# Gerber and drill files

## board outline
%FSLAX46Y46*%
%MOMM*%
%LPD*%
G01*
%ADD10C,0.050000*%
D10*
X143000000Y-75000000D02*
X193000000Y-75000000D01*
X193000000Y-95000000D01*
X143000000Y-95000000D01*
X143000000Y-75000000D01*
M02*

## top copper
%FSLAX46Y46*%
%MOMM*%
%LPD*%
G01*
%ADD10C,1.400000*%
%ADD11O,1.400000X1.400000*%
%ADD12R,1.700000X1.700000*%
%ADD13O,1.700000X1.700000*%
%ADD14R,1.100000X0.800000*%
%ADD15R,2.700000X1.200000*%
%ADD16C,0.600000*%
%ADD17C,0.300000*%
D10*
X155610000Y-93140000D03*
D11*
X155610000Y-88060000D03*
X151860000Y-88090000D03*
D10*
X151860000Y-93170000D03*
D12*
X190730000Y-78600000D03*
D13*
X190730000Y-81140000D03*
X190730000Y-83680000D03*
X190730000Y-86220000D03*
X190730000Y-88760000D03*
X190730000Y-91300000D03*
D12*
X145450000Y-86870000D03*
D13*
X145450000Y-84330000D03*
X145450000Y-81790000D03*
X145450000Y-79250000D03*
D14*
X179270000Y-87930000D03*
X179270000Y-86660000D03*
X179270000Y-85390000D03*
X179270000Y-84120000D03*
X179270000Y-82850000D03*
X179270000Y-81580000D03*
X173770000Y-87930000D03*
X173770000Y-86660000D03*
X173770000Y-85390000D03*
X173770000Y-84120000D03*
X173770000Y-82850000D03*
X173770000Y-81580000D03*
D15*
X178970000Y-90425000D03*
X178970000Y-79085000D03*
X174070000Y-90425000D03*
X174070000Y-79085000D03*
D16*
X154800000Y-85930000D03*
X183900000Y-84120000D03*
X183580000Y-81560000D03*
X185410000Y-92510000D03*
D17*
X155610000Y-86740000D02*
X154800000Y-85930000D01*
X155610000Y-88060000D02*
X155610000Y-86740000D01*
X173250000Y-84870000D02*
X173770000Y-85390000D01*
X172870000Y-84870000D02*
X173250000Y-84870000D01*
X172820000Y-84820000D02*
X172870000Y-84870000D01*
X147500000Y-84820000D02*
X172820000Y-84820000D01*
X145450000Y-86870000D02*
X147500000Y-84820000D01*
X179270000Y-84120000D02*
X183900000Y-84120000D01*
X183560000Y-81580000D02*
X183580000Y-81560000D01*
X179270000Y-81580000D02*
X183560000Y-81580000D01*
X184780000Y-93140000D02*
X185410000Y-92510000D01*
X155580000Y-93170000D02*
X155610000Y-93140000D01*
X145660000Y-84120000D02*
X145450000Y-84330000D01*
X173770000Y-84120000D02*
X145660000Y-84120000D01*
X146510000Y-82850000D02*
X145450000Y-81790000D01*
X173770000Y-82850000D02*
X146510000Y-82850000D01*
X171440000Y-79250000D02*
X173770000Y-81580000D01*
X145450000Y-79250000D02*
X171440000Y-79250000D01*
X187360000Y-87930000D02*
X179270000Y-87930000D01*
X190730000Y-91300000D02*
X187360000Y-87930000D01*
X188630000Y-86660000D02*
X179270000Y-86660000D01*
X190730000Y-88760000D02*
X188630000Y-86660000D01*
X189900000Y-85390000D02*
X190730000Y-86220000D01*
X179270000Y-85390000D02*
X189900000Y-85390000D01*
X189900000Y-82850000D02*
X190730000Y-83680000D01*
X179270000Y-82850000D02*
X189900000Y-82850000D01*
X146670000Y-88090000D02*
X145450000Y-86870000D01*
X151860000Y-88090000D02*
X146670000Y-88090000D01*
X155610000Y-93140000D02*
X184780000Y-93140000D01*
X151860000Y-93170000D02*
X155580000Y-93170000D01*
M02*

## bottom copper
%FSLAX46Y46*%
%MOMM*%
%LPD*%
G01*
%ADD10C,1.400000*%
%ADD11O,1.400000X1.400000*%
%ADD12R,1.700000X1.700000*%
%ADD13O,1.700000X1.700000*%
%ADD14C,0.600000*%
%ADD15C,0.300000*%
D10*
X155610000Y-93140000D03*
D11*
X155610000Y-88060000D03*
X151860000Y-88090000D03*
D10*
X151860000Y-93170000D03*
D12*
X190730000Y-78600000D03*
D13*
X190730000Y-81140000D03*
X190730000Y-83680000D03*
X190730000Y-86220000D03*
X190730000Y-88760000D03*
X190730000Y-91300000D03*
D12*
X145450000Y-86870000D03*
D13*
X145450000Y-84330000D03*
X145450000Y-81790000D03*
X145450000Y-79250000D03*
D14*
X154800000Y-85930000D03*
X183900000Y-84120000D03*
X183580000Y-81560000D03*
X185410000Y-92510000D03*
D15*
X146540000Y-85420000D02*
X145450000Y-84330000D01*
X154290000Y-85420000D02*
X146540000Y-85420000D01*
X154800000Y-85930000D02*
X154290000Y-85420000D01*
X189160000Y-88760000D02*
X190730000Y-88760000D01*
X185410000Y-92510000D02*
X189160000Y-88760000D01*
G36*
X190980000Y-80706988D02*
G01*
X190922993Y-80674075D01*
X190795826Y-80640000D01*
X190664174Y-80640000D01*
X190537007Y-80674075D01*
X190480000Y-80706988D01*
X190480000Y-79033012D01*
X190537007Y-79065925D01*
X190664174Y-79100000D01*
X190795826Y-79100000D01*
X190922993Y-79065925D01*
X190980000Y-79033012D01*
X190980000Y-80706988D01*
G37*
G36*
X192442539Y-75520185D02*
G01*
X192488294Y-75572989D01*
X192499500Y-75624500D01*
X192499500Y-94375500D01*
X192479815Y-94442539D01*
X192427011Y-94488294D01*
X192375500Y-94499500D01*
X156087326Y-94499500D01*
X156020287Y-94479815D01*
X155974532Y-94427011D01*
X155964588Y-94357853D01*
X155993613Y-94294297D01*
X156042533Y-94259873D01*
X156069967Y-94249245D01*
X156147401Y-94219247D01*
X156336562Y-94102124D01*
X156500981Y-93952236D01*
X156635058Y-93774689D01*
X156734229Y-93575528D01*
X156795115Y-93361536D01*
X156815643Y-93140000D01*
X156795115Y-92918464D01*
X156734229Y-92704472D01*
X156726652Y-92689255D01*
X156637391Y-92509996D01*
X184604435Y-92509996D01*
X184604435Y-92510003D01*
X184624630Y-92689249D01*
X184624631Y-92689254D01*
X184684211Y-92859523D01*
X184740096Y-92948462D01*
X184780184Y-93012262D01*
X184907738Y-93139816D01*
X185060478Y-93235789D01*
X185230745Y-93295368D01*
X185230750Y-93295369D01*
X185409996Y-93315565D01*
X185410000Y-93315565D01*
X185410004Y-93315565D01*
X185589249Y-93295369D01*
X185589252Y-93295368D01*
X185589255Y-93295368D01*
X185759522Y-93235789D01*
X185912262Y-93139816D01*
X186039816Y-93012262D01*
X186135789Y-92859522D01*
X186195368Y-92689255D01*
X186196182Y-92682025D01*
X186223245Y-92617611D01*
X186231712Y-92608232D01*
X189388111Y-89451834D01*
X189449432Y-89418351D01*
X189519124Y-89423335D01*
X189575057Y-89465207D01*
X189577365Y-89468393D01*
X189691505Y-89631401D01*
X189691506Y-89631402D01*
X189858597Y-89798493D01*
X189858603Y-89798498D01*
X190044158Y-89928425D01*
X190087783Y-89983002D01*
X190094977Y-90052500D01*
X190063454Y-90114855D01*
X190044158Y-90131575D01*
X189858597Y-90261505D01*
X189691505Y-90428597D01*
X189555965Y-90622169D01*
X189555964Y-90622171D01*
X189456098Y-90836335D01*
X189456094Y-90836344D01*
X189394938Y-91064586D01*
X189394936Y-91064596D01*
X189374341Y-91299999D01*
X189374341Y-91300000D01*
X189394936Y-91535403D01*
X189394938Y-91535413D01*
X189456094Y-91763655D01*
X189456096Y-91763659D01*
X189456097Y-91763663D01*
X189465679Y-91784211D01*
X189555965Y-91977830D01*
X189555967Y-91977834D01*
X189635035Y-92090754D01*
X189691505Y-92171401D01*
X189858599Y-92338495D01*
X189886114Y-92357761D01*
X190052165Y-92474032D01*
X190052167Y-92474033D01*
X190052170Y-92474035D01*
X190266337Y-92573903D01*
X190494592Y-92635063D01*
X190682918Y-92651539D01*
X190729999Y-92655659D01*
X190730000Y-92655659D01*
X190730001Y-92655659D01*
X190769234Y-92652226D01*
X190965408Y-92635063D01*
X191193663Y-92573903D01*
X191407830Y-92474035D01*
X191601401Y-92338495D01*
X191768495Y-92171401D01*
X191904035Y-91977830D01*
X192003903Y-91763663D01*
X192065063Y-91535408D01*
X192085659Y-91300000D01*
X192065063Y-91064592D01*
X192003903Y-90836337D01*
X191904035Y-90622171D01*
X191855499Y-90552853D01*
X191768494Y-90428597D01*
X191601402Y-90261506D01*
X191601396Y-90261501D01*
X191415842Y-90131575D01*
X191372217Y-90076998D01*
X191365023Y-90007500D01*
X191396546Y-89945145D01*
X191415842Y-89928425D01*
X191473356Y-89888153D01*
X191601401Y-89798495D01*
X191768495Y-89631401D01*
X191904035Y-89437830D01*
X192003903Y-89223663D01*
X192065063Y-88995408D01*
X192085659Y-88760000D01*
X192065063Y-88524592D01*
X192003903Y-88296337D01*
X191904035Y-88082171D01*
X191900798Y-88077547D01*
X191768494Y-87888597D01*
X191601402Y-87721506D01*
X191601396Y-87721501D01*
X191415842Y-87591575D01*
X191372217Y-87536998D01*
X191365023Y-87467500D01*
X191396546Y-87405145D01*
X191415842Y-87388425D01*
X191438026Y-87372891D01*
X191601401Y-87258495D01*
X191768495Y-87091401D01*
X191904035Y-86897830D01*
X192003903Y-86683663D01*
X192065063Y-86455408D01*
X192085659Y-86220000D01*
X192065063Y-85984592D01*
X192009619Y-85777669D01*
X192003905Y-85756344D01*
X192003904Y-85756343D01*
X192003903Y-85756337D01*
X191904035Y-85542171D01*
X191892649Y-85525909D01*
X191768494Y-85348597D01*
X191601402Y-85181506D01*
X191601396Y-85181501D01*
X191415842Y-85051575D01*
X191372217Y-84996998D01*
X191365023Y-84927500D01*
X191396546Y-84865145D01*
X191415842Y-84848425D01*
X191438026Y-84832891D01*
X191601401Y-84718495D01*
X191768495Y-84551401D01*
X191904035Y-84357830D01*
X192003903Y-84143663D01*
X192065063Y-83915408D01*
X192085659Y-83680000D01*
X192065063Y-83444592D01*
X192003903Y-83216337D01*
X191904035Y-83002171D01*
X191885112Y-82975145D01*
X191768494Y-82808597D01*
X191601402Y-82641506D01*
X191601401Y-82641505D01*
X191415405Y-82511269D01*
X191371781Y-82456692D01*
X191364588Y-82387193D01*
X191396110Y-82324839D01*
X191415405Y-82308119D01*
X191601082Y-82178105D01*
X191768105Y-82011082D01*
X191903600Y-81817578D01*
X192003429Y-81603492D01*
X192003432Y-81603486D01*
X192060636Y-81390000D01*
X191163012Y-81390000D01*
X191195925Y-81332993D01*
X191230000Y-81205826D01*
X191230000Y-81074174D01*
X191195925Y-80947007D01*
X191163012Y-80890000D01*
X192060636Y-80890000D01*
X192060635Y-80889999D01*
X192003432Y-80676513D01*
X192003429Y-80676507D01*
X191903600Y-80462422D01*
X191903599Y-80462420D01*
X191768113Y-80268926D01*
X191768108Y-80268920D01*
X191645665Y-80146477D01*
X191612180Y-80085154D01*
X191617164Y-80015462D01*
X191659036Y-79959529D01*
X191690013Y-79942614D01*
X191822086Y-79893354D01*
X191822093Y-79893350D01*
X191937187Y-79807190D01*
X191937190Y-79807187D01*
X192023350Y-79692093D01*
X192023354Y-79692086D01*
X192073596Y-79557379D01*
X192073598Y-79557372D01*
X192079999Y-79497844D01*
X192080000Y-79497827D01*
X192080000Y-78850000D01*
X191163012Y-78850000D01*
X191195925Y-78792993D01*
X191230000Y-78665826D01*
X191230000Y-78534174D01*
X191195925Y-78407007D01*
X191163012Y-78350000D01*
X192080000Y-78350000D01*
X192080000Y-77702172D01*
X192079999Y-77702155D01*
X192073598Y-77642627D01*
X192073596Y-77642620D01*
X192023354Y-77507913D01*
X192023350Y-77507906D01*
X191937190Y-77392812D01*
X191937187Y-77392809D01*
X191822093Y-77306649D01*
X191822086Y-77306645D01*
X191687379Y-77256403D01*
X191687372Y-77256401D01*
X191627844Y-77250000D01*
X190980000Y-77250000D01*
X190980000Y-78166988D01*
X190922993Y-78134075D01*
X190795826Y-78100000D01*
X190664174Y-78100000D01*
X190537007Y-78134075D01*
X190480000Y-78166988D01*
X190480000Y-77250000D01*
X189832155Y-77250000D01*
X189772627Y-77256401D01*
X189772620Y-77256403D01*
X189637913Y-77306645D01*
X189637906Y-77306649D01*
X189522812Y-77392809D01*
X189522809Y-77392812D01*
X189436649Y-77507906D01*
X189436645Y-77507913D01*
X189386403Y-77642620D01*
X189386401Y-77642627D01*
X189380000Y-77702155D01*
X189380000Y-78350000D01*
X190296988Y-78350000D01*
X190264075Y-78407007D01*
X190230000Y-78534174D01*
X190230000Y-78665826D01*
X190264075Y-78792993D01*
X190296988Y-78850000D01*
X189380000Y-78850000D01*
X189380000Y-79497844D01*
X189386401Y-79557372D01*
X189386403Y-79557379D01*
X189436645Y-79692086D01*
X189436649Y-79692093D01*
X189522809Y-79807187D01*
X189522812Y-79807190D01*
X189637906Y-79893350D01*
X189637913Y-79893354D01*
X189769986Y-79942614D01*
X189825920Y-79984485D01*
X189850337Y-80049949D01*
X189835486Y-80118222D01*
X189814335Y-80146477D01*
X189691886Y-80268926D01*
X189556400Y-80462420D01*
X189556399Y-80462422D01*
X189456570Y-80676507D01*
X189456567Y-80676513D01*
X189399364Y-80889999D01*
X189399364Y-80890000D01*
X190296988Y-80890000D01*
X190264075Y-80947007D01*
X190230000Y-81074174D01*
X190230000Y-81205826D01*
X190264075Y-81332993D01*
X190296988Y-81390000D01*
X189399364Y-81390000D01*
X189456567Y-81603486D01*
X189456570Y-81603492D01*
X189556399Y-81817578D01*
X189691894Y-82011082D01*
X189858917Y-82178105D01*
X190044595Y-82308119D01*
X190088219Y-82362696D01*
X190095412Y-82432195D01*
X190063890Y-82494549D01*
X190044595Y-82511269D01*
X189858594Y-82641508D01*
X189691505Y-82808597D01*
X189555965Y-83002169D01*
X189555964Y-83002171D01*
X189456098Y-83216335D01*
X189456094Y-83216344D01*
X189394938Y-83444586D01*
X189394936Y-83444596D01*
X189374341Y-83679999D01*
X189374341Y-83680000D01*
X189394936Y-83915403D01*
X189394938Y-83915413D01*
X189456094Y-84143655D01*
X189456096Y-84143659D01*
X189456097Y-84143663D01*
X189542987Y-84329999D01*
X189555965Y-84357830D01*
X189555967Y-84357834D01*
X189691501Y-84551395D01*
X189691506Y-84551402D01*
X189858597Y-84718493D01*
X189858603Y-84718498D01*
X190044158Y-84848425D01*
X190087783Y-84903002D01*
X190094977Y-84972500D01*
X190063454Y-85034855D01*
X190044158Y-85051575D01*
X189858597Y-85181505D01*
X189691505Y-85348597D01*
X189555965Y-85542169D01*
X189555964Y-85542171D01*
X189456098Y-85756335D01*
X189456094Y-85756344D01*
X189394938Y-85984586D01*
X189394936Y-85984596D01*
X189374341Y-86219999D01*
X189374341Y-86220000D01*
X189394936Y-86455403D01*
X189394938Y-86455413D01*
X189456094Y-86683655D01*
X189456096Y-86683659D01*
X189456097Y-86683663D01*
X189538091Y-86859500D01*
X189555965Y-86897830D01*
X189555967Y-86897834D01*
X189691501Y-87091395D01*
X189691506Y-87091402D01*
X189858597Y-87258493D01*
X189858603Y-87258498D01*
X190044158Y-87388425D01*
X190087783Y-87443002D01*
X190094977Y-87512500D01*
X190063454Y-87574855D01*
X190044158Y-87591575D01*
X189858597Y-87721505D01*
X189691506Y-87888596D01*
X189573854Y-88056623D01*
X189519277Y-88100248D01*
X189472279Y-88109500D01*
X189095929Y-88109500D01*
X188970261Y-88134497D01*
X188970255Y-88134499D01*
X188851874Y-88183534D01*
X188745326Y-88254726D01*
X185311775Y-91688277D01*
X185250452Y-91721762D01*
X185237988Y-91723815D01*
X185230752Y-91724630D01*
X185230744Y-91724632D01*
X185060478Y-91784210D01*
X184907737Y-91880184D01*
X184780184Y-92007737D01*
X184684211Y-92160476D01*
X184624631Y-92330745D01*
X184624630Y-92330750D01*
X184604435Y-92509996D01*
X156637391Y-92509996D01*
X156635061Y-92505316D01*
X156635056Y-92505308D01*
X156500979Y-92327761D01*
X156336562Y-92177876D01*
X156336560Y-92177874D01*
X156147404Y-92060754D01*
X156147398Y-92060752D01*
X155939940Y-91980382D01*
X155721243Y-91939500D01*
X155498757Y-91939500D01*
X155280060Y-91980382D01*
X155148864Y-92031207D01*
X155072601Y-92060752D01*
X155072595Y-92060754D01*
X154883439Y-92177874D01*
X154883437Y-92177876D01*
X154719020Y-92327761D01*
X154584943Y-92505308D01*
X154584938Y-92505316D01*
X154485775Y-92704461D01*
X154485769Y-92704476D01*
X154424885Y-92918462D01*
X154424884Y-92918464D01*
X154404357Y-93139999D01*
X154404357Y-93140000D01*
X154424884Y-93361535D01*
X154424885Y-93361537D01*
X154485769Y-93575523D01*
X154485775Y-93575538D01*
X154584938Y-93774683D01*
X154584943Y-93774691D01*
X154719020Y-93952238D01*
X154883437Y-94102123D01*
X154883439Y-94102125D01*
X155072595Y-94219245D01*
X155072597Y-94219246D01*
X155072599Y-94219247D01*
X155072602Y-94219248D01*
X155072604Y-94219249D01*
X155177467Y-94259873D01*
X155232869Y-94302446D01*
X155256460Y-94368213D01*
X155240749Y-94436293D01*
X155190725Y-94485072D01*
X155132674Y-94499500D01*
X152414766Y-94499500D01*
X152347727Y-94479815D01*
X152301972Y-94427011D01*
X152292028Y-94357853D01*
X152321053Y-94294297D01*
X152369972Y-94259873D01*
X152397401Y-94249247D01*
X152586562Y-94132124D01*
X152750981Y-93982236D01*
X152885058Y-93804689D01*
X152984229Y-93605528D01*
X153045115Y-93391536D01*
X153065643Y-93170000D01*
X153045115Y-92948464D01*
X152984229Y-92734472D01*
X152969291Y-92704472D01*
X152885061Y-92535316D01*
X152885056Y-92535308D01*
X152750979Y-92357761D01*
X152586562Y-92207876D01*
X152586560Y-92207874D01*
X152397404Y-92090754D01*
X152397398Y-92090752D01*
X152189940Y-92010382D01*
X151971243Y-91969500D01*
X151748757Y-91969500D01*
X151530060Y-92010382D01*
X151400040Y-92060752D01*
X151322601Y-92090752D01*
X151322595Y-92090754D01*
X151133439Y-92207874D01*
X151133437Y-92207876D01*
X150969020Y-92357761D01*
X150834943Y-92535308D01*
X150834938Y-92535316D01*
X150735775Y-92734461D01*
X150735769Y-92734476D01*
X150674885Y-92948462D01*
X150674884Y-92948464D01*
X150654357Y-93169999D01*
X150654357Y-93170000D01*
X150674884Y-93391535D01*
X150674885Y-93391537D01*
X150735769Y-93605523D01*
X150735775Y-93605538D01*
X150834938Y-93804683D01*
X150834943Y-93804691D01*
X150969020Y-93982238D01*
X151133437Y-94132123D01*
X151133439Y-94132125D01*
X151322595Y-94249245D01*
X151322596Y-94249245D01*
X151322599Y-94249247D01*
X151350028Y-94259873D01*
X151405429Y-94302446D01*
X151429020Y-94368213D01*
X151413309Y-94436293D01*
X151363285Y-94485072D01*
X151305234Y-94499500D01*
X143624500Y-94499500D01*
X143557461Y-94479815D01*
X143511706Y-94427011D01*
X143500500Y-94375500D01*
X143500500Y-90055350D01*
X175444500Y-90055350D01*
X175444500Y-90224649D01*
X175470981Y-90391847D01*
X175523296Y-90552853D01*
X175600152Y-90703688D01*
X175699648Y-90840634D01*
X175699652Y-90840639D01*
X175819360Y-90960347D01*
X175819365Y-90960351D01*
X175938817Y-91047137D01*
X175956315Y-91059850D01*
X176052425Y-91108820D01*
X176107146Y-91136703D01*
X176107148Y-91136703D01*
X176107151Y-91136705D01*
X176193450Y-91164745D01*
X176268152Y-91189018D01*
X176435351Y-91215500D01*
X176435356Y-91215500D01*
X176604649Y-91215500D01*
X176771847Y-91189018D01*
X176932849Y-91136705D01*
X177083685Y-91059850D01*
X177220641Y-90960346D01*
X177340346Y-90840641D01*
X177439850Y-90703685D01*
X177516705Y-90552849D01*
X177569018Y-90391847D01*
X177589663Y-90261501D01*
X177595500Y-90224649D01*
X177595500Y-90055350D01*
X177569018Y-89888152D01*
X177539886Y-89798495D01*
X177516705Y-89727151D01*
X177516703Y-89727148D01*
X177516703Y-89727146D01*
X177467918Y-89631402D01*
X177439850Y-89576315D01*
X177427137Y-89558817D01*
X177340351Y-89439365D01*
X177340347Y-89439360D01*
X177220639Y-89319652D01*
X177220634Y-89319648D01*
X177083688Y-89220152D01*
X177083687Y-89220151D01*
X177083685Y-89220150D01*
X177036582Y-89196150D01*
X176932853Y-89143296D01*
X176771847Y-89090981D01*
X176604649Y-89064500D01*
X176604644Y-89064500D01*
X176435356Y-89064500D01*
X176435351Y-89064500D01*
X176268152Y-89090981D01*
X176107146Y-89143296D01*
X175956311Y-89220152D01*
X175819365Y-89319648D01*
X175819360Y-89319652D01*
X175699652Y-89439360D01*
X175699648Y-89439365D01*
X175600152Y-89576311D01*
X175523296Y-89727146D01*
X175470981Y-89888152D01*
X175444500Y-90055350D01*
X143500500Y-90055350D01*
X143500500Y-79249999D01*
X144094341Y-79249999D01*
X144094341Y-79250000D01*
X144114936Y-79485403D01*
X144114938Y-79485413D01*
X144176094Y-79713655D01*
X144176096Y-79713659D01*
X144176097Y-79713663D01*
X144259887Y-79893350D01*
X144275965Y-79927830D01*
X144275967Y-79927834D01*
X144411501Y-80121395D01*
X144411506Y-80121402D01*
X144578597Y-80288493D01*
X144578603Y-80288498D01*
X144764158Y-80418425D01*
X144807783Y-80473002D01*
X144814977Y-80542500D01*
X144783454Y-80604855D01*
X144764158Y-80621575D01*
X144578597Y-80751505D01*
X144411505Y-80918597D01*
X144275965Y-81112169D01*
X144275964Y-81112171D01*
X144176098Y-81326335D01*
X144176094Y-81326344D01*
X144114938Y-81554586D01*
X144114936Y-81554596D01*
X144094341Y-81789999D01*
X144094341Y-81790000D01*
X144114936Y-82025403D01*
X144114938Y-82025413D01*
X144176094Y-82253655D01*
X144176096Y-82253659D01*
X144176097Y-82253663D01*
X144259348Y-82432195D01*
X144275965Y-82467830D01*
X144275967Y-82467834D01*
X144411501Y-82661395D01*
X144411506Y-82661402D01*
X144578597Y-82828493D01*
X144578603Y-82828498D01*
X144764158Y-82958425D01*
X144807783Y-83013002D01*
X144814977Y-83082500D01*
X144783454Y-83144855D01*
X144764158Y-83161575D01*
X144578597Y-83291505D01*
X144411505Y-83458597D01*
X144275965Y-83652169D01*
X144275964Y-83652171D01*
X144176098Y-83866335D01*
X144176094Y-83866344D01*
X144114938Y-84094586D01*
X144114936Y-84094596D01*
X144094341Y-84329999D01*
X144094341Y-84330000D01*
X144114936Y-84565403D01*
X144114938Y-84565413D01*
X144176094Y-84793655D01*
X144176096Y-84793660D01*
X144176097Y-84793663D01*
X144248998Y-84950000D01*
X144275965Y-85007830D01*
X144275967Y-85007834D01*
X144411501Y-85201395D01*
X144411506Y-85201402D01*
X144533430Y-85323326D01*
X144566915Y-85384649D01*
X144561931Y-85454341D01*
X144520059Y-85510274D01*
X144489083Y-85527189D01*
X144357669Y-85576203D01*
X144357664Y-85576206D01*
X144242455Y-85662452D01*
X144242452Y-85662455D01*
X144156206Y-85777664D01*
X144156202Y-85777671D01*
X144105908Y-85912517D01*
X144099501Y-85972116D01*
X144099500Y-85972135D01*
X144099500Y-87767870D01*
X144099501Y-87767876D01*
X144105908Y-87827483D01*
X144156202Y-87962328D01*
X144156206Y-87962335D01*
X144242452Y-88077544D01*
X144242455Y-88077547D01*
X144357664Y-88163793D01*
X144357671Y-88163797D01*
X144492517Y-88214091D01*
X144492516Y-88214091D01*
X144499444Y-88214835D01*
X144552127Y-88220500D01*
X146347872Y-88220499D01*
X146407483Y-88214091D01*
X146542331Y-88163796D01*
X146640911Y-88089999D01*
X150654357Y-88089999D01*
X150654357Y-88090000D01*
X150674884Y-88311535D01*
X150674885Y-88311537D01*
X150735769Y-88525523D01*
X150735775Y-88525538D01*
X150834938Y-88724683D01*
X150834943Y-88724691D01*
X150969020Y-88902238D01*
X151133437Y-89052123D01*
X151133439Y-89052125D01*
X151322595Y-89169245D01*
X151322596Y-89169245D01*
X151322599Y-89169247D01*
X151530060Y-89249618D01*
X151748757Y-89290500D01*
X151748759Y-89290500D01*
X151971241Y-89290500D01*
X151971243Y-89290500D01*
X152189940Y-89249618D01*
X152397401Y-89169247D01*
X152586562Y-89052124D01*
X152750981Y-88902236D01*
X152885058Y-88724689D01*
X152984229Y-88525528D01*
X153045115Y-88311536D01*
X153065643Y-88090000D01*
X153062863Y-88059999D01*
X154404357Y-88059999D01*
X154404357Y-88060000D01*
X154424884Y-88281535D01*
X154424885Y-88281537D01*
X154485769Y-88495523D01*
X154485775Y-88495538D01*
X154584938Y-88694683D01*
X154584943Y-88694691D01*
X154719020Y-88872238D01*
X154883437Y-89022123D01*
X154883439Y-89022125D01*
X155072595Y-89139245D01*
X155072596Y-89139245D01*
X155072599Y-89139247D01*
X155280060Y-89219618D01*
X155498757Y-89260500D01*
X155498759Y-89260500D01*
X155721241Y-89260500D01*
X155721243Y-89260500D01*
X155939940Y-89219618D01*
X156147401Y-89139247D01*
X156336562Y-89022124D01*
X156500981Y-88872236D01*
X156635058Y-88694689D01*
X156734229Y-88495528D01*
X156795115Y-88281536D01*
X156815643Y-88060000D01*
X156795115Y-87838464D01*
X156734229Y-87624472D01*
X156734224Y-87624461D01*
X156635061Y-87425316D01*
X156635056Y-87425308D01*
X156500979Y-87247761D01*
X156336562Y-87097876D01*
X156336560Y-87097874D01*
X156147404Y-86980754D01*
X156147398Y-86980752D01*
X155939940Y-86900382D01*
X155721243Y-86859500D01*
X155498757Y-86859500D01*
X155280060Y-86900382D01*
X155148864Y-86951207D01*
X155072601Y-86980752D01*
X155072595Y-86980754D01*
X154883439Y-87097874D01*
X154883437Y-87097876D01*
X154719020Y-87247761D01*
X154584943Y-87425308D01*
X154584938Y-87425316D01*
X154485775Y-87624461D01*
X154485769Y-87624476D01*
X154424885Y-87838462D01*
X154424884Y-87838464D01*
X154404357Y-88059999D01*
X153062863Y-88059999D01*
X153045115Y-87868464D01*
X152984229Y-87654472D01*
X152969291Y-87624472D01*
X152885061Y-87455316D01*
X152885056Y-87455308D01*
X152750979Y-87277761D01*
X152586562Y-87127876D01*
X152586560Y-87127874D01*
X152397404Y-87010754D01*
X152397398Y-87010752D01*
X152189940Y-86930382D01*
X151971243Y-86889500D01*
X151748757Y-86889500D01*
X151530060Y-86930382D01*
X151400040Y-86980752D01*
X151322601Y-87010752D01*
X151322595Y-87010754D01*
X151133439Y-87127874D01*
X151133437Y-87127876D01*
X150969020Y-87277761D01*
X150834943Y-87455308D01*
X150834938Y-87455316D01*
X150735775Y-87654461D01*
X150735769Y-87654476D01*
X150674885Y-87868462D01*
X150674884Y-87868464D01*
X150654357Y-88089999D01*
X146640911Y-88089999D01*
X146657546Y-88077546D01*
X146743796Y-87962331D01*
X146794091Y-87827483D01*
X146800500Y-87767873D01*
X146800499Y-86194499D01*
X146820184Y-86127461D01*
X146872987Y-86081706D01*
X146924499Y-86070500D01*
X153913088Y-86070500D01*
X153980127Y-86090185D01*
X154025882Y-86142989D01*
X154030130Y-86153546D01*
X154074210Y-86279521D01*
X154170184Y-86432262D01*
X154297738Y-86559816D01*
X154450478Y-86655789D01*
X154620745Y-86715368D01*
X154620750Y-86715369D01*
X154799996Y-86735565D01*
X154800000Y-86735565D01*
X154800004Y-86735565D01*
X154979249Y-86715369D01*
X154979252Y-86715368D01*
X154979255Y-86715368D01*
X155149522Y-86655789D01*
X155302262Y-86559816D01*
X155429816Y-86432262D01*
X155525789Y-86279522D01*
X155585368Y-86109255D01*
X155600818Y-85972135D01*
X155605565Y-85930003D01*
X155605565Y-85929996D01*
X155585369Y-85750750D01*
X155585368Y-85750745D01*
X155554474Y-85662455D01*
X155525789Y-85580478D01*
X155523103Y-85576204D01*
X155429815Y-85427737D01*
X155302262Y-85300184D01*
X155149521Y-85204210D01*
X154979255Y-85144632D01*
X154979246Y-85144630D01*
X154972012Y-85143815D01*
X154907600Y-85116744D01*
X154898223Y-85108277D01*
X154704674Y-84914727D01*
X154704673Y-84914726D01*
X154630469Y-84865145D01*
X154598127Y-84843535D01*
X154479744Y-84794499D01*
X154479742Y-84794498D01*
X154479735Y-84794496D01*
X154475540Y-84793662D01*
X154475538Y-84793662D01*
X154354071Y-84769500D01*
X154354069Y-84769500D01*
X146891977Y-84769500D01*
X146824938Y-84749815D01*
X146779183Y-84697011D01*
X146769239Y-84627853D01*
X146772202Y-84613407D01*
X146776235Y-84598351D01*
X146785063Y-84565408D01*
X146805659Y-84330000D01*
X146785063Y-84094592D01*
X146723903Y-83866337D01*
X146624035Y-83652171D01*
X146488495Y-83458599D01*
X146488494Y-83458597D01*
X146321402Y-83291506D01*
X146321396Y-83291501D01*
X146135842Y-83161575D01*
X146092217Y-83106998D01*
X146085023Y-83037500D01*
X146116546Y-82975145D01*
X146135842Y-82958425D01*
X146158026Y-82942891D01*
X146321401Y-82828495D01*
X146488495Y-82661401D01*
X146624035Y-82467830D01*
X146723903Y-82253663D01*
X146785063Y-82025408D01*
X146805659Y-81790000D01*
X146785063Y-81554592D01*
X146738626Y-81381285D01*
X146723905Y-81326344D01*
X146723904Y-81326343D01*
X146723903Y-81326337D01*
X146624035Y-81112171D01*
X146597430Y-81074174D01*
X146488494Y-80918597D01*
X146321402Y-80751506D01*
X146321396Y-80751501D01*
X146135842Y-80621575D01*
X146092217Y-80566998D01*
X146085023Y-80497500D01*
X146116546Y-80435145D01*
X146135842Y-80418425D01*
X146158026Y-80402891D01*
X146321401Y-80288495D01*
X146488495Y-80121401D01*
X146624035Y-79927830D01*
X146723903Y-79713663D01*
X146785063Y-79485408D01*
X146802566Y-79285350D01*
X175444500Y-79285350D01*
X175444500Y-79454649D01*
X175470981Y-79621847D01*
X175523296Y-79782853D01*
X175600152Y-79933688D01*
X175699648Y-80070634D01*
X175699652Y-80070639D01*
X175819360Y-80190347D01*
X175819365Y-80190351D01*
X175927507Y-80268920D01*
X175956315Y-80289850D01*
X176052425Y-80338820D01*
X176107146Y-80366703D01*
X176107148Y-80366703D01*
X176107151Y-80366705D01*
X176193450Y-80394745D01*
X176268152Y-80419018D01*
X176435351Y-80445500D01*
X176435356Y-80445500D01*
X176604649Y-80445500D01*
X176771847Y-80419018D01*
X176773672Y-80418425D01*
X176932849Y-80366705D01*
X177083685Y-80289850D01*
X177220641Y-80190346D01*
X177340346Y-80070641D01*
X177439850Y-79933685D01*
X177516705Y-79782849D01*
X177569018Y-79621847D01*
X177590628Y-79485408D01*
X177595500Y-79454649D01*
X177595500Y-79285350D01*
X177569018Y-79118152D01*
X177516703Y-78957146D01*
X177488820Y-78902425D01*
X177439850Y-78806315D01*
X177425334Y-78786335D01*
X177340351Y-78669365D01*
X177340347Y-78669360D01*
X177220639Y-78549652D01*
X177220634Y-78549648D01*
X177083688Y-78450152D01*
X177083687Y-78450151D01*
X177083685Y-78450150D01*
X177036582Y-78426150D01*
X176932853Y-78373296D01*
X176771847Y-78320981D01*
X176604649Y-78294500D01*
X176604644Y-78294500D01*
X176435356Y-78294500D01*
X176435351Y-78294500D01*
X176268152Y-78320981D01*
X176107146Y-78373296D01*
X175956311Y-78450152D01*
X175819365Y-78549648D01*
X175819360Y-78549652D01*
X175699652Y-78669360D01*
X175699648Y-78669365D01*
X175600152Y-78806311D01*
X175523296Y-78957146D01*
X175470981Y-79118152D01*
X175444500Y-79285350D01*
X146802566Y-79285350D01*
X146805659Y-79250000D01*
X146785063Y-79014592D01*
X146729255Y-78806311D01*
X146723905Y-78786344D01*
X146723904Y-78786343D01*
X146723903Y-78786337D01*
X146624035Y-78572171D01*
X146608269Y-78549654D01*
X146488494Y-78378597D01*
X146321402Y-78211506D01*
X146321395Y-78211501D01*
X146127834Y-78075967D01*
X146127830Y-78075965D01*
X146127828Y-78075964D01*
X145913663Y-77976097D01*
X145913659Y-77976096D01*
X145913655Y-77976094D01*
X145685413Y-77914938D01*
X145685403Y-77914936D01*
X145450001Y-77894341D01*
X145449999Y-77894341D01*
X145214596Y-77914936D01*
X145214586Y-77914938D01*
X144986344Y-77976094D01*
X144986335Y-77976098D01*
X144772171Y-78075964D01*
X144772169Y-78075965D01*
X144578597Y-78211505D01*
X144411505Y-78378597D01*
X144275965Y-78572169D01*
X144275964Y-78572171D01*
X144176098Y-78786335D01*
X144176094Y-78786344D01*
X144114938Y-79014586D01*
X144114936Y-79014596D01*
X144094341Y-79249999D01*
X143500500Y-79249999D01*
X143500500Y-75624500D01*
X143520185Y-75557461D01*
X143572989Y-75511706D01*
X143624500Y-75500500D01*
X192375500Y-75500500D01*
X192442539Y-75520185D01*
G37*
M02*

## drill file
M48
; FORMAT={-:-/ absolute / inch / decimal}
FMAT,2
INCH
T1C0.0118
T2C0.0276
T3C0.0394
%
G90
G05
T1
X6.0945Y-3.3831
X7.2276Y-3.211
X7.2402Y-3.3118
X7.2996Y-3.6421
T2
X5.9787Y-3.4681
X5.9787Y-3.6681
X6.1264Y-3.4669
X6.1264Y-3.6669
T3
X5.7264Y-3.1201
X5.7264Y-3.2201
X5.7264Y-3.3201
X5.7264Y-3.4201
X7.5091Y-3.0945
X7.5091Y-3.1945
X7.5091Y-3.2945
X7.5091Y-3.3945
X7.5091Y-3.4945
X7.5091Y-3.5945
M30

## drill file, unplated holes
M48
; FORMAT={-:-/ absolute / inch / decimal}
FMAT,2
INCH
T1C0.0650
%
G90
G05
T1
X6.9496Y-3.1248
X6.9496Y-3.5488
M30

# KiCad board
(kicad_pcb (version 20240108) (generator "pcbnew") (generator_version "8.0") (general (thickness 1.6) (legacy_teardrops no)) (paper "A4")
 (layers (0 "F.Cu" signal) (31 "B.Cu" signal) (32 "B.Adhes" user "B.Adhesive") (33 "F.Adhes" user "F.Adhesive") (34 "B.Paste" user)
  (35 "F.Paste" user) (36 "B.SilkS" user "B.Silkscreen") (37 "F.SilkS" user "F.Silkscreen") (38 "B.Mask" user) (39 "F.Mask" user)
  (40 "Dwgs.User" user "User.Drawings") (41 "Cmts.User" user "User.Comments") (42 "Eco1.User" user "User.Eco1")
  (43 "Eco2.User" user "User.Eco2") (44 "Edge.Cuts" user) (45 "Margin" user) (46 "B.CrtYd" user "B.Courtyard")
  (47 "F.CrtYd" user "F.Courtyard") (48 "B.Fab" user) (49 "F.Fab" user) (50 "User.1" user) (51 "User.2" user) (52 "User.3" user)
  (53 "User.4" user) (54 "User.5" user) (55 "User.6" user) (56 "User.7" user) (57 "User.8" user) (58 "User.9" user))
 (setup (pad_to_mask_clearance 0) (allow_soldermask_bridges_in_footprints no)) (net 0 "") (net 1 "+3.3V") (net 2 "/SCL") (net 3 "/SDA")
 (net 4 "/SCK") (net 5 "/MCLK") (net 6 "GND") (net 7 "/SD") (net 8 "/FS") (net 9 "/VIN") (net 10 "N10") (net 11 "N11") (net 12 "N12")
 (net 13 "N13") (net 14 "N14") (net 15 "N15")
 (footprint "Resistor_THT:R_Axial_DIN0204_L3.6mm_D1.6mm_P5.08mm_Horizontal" (layer "F.Cu") (at 151.86 93.17 90)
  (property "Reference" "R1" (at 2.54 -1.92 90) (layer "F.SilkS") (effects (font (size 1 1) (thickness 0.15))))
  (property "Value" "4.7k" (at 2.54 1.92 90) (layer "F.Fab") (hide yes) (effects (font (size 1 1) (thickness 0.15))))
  (pad "1" thru_hole circle (at 0 0 90) (size 1.4 1.4) (drill 0.7) (layers "*.Cu" "*.Mask") (remove_unused_layers no) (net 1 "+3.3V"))
  (pad "2" thru_hole oval (at 5.08 0 90) (size 1.4 1.4) (drill 0.7) (layers "*.Cu" "*.Mask") (remove_unused_layers no) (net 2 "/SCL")))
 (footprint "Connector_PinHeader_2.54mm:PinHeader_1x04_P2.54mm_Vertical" (layer "F.Cu") (at 145.45 86.87 180)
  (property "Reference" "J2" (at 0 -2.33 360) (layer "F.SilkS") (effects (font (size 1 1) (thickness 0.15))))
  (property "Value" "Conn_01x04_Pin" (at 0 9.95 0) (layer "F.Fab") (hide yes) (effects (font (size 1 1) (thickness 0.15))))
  (pad "1" thru_hole rect (at 0 0 180) (size 1.7 1.7) (drill 1) (layers "*.Cu" "*.Mask") (remove_unused_layers no) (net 2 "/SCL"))
  (pad "2" thru_hole oval (at 0 2.54 180) (size 1.7 1.7) (drill 1) (layers "*.Cu" "*.Mask") (remove_unused_layers no) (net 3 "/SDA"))
  (pad "3" thru_hole oval (at 0 5.08 180) (size 1.7 1.7) (drill 1) (layers "*.Cu" "*.Mask") (remove_unused_layers no) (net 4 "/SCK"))
  (pad "4" thru_hole oval (at 0 7.62 180) (size 1.7 1.7) (drill 1) (layers "*.Cu" "*.Mask") (remove_unused_layers no) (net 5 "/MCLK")))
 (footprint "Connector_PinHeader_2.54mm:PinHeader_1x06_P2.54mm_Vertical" (layer "F.Cu") (at 190.73 78.6)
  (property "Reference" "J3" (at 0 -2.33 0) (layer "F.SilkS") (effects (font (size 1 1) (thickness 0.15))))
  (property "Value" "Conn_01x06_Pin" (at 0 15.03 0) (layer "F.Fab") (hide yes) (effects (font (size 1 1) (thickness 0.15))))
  (pad "1" thru_hole rect (at 0 0) (size 1.7 1.7) (drill 1) (layers "*.Cu" "*.Mask") (remove_unused_layers no) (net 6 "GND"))
  (pad "2" thru_hole oval (at 0 2.54) (size 1.7 1.7) (drill 1) (layers "*.Cu" "*.Mask") (remove_unused_layers no) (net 6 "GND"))
  (pad "3" thru_hole oval (at 0 5.08) (size 1.7 1.7) (drill 1) (layers "*.Cu" "*.Mask") (remove_unused_layers no) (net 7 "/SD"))
  (pad "4" thru_hole oval (at 0 7.62) (size 1.7 1.7) (drill 1) (layers "*.Cu" "*.Mask") (remove_unused_layers no) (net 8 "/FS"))
  (pad "5" thru_hole oval (at 0 10.16) (size 1.7 1.7) (drill 1) (layers "*.Cu" "*.Mask") (remove_unused_layers no) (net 1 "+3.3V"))
  (pad "6" thru_hole oval (at 0 12.7) (size 1.7 1.7) (drill 1) (layers "*.Cu" "*.Mask") (remove_unused_layers no) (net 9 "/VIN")))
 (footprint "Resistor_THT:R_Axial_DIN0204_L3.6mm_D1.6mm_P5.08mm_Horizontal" (layer "F.Cu") (at 155.61 93.14 90)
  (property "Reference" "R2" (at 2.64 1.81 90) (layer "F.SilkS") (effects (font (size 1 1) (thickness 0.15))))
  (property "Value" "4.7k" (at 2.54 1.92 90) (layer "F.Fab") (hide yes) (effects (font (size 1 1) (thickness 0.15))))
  (pad "1" thru_hole circle (at 0 0 90) (size 1.4 1.4) (drill 0.7) (layers "*.Cu" "*.Mask") (remove_unused_layers no) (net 1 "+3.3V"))
  (pad "2" thru_hole oval (at 5.08 0 90) (size 1.4 1.4) (drill 0.7) (layers "*.Cu" "*.Mask") (remove_unused_layers no) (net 3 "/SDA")))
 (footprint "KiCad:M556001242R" (layer "F.Cu") (at 176.52 84.755 90)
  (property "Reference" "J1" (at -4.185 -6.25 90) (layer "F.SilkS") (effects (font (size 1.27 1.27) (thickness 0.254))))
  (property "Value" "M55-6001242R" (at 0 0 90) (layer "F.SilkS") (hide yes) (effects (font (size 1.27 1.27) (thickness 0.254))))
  (pad "" np_thru_hole circle (at -5.385 0 90) (size 1.65 1.65) (drill 1.65) (layers "*.Cu" "*.Mask"))
  (pad "" np_thru_hole circle (at 5.385 0 90) (size 1.65 1.65) (drill 1.65) (layers "*.Cu" "*.Mask"))
  (pad "A1" smd rect (at -3.175 2.75 90) (size 0.8 1.1) (layers "F.Cu" "F.Paste" "F.Mask") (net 9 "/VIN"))
  (pad "A2" smd rect (at -1.905 2.75 90) (size 0.8 1.1) (layers "F.Cu" "F.Paste" "F.Mask") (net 1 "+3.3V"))
  (pad "A3" smd rect (at -0.635 2.75 90) (size 0.8 1.1) (layers "F.Cu" "F.Paste" "F.Mask") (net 8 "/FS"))
  (pad "A4" smd rect (at 0.635 2.75 90) (size 0.8 1.1) (layers "F.Cu" "F.Paste" "F.Mask") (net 6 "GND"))
  (pad "A5" smd rect (at 1.905 2.75 90) (size 0.8 1.1) (layers "F.Cu" "F.Paste" "F.Mask") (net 7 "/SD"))
  (pad "A6" smd rect (at 3.175 2.75 90) (size 0.8 1.1) (layers "F.Cu" "F.Paste" "F.Mask") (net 6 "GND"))
  (pad "B1" smd rect (at -3.175 -2.75 90) (size 0.8 1.1) (layers "F.Cu" "F.Paste" "F.Mask") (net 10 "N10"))
  (pad "B2" smd rect (at -1.905 -2.75 90) (size 0.8 1.1) (layers "F.Cu" "F.Paste" "F.Mask") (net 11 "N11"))
  (pad "B3" smd rect (at -0.635 -2.75 90) (size 0.8 1.1) (layers "F.Cu" "F.Paste" "F.Mask") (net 2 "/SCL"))
  (pad "B4" smd rect (at 0.635 -2.75 90) (size 0.8 1.1) (layers "F.Cu" "F.Paste" "F.Mask") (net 3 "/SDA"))
  (pad "B5" smd rect (at 1.905 -2.75 90) (size 0.8 1.1) (layers "F.Cu" "F.Paste" "F.Mask") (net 4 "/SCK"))
  (pad "B6" smd rect (at 3.175 -2.75 90) (size 0.8 1.1) (layers "F.Cu" "F.Paste" "F.Mask") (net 5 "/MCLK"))
  (pad "MP1" smd rect (at -5.67 2.45 90) (size 1.2 2.7) (layers "F.Cu" "F.Paste" "F.Mask") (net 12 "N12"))
  (pad "MP2" smd rect (at 5.67 2.45 90) (size 1.2 2.7) (layers "F.Cu" "F.Paste" "F.Mask") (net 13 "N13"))
  (pad "MP3" smd rect (at -5.67 -2.45 90) (size 1.2 2.7) (layers "F.Cu" "F.Paste" "F.Mask") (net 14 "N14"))
  (pad "MP4" smd rect (at 5.67 -2.45 90) (size 1.2 2.7) (layers "F.Cu" "F.Paste" "F.Mask") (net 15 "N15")))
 (gr_rect (start 143 75) (end 193 95) (stroke (width 0.05) (type default)) (fill none) (layer "Edge.Cuts"))
 (segment (start 146.51 82.85) (end 145.45 81.79) (width 0.3) (layer "F.Cu") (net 4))
 (segment (start 173.77 82.85) (end 146.51 82.85) (width 0.3) (layer "F.Cu") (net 4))
 (segment (start 179.27 81.58) (end 183.56 81.58) (width 0.3) (layer "F.Cu") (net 6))
 (segment (start 179.27 84.12) (end 183.9 84.12) (width 0.3) (layer "F.Cu") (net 6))
 (segment (start 183.56 81.58) (end 183.58 81.56) (width 0.3) (layer "F.Cu") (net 6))
 (via (at 183.9 84.12) (size 0.6) (drill 0.3) (layers "F.Cu" "B.Cu") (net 6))
 (via (at 183.58 81.56) (size 0.6) (drill 0.3) (layers "F.Cu" "B.Cu") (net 6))
 (segment (start 187.36 87.93) (end 179.27 87.93) (width 0.3) (layer "F.Cu") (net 9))
 (segment (start 190.73 91.3) (end 187.36 87.93) (width 0.3) (layer "F.Cu") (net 9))
 (segment (start 189.9 85.39) (end 190.73 86.22) (width 0.3) (layer "F.Cu") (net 8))
 (segment (start 179.27 85.39) (end 189.9 85.39) (width 0.3) (layer "F.Cu") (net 8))
 (segment (start 155.61 88.06) (end 155.61 86.74) (width 0.3) (layer "F.Cu") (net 3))
 (segment (start 155.61 86.74) (end 154.8 85.93) (width 0.3) (layer "F.Cu") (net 3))
 (segment (start 145.66 84.12) (end 145.45 84.33) (width 0.3) (layer "F.Cu") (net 3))
 (segment (start 173.77 84.12) (end 145.66 84.12) (width 0.3) (layer "F.Cu") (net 3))
 (via (at 154.8 85.93) (size 0.6) (drill 0.3) (layers "F.Cu" "B.Cu") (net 3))
 (segment (start 154.29 85.42) (end 146.54 85.42) (width 0.3) (layer "B.Cu") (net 3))
 (segment (start 154.8 85.93) (end 154.29 85.42) (width 0.3) (layer "B.Cu") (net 3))
 (segment (start 146.54 85.42) (end 145.45 84.33) (width 0.3) (layer "B.Cu") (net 3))
 (segment (start 172.87 84.87) (end 173.25 84.87) (width 0.3) (layer "F.Cu") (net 2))
 (segment (start 151.86 88.09) (end 146.67 88.09) (width 0.3) (layer "F.Cu") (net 2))
 (segment (start 172.82 84.82) (end 172.87 84.87) (width 0.3) (layer "F.Cu") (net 2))
 (segment (start 147.5 84.82) (end 172.82 84.82) (width 0.3) (layer "F.Cu") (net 2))
 (segment (start 145.45 86.87) (end 147.5 84.82) (width 0.3) (layer "F.Cu") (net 2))
 (segment (start 173.25 84.87) (end 173.77 85.39) (width 0.3) (layer "F.Cu") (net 2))
 (segment (start 146.67 88.09) (end 145.45 86.87) (width 0.3) (layer "F.Cu") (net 2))
 (segment (start 155.58 93.17) (end 155.61 93.14) (width 0.3) (layer "F.Cu") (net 1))
 (segment (start 188.63 86.66) (end 179.27 86.66) (width 0.3) (layer "F.Cu") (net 1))
 (segment (start 151.86 93.17) (end 155.58 93.17) (width 0.3) (layer "F.Cu") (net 1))
 (segment (start 184.78 93.14) (end 185.41 92.51) (width 0.3) (layer "F.Cu") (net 1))
 (segment (start 155.61 93.14) (end 184.78 93.14) (width 0.3) (layer "F.Cu") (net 1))
 (segment (start 190.73 88.76) (end 188.63 86.66) (width 0.3) (layer "F.Cu") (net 1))
 (via (at 185.41 92.51) (size 0.6) (drill 0.3) (layers "F.Cu" "B.Cu") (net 1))
 (segment (start 185.41 92.51) (end 189.16 88.76) (width 0.3) (layer "B.Cu") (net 1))
 (segment (start 189.16 88.76) (end 190.73 88.76) (width 0.3) (layer "B.Cu") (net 1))
 (segment (start 145.45 79.25) (end 171.44 79.25) (width 0.3) (layer "F.Cu") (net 5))
 (segment (start 171.44 79.25) (end 173.77 81.58) (width 0.3) (layer "F.Cu") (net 5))
 (segment (start 189.9 82.85) (end 190.73 83.68) (width 0.3) (layer "F.Cu") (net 7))
 (segment (start 179.27 82.85) (end 189.9 82.85) (width 0.3) (layer "F.Cu") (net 7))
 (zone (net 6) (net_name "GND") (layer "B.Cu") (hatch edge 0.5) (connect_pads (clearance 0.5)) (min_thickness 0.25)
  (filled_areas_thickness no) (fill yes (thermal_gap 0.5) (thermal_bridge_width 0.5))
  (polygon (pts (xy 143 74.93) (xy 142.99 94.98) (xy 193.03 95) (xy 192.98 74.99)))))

